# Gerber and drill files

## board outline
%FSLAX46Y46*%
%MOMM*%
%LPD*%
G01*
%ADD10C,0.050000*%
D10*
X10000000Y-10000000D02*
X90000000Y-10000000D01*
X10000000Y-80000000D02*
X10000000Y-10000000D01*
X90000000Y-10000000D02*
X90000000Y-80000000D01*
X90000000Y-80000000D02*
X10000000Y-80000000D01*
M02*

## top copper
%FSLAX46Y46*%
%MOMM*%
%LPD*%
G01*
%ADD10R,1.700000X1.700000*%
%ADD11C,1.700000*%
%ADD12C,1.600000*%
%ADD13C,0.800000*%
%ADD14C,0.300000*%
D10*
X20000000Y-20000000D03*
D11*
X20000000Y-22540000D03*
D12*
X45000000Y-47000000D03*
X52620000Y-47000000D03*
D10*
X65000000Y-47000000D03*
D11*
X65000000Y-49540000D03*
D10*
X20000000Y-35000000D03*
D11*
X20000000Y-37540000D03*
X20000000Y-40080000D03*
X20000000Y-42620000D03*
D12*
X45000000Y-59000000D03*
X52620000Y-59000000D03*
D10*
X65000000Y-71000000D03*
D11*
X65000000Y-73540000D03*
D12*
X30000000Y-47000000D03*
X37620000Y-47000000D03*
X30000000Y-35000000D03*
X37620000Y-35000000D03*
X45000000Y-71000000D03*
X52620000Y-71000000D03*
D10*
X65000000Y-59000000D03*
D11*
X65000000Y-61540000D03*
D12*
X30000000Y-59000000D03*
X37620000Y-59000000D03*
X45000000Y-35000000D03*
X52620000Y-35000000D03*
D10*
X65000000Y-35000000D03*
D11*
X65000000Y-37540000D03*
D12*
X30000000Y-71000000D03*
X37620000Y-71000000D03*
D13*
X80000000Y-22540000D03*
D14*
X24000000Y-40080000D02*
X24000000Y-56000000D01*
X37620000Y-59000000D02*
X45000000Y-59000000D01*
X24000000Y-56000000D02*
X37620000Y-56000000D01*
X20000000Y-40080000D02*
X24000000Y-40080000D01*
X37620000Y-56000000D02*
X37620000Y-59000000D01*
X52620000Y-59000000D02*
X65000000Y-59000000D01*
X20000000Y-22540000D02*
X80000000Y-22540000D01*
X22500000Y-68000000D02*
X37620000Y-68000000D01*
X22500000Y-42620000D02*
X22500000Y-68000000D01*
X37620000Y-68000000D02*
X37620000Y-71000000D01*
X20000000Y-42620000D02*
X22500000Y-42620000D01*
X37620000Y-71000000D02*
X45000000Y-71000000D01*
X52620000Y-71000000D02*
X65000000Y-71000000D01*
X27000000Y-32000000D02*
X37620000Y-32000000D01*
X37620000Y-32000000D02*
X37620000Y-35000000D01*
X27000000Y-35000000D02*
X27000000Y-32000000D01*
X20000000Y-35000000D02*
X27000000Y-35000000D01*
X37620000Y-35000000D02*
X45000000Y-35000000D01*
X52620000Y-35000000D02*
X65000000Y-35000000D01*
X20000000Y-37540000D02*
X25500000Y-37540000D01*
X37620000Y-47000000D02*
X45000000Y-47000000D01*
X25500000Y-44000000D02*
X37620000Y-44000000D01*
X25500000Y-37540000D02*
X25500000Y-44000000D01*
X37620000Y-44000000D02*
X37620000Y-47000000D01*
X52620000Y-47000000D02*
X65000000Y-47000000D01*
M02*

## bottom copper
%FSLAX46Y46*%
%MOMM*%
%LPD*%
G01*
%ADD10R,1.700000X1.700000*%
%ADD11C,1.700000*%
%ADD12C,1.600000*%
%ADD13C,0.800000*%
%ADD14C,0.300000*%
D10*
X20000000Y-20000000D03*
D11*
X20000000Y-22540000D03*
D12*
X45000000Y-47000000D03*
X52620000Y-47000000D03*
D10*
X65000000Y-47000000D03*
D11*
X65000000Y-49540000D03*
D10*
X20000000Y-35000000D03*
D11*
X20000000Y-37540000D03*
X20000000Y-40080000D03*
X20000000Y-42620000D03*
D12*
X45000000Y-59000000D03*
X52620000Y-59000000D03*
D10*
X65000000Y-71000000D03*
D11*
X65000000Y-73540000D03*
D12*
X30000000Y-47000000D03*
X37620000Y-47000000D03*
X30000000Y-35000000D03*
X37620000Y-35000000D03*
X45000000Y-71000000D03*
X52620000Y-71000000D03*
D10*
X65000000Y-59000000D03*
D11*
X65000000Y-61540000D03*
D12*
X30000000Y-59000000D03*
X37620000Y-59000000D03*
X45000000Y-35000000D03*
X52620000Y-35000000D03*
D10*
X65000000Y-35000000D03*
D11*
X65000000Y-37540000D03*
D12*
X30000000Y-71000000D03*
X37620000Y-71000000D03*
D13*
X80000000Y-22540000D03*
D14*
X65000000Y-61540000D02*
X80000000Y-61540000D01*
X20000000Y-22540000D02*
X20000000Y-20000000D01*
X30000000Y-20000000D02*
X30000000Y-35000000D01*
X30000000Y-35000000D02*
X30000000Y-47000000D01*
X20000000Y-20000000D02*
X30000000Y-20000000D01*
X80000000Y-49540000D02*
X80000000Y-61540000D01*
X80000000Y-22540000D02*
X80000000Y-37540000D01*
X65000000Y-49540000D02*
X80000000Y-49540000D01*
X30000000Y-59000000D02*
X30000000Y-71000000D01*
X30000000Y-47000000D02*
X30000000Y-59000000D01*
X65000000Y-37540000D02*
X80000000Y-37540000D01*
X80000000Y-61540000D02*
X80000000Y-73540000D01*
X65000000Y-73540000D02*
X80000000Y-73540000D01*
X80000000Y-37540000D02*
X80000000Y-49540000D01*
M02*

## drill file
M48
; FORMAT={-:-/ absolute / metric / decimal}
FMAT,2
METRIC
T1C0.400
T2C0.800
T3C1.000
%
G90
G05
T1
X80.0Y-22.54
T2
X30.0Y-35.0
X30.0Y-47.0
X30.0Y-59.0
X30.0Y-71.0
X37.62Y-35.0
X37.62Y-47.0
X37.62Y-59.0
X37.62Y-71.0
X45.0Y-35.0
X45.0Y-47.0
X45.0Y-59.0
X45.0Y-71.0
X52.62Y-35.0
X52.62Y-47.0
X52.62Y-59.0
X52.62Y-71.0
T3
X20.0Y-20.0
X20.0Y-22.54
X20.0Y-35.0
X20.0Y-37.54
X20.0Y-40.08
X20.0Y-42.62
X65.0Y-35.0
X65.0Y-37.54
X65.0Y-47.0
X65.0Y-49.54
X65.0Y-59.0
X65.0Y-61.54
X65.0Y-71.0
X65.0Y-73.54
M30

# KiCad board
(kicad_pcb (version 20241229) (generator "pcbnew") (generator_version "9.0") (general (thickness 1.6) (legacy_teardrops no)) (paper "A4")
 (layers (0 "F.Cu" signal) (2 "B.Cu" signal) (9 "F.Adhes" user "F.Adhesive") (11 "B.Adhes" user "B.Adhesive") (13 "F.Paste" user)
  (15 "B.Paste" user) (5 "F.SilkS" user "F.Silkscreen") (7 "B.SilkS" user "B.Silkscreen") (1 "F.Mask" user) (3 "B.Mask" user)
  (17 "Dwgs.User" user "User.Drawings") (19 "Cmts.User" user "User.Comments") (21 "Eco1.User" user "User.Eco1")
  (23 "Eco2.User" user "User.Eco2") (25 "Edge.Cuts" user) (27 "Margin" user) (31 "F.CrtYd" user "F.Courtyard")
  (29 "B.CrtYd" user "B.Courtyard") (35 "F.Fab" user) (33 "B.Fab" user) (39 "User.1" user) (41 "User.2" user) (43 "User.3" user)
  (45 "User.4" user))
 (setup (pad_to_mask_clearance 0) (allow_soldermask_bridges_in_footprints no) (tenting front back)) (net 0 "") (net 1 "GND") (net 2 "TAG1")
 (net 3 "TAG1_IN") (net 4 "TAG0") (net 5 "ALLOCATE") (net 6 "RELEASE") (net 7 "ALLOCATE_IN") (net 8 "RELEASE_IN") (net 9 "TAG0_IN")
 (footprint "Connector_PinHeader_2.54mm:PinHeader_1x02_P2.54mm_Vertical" (layer "F.Cu") (at 20 20)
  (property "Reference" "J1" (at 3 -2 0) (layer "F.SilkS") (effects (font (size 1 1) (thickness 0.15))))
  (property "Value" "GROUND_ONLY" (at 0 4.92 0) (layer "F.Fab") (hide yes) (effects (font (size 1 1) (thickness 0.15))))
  (pad "1" thru_hole rect (at 0 0) (size 1.7 1.7) (drill 1) (layers "*.Cu" "*.Mask") (remove_unused_layers no) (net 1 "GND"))
  (pad "2" thru_hole circle (at 0 2.54) (size 1.7 1.7) (drill 1) (layers "*.Cu" "*.Mask") (remove_unused_layers no) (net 1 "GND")))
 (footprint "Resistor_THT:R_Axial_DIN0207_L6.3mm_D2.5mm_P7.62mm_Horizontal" (layer "F.Cu") (at 45 47)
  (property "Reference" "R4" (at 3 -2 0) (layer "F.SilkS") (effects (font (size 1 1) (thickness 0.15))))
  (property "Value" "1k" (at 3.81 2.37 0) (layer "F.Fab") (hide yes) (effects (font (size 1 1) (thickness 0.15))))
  (pad "1" thru_hole circle (at 0 0) (size 1.6 1.6) (drill 0.8) (layers "*.Cu" "*.Mask") (remove_unused_layers no) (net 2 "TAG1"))
  (pad "2" thru_hole circle (at 7.62 0) (size 1.6 1.6) (drill 0.8) (layers "*.Cu" "*.Mask") (remove_unused_layers no) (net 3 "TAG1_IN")))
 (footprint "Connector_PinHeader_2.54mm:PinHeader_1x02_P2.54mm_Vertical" (layer "F.Cu") (at 65 47)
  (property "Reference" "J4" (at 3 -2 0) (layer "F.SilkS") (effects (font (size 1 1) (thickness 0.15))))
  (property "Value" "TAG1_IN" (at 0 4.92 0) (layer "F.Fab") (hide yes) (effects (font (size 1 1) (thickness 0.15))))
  (pad "1" thru_hole rect (at 0 0) (size 1.7 1.7) (drill 1) (layers "*.Cu" "*.Mask") (remove_unused_layers no) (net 3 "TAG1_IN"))
  (pad "2" thru_hole circle (at 0 2.54) (size 1.7 1.7) (drill 1) (layers "*.Cu" "*.Mask") (remove_unused_layers no) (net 1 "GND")))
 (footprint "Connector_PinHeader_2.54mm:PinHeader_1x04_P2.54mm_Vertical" (layer "F.Cu") (at 20 35)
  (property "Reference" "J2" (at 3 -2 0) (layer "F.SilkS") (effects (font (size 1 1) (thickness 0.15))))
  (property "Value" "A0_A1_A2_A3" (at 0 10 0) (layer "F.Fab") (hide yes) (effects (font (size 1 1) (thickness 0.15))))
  (pad "1" thru_hole rect (at 0 0) (size 1.7 1.7) (drill 1) (layers "*.Cu" "*.Mask") (remove_unused_layers no) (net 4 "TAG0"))
  (pad "2" thru_hole circle (at 0 2.54) (size 1.7 1.7) (drill 1) (layers "*.Cu" "*.Mask") (remove_unused_layers no) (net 2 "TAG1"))
  (pad "3" thru_hole circle (at 0 5.08) (size 1.7 1.7) (drill 1) (layers "*.Cu" "*.Mask") (remove_unused_layers no) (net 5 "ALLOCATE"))
  (pad "4" thru_hole circle (at 0 7.62) (size 1.7 1.7) (drill 1) (layers "*.Cu" "*.Mask") (remove_unused_layers no) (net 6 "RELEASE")))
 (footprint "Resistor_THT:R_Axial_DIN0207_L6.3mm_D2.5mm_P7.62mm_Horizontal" (layer "F.Cu") (at 45 59)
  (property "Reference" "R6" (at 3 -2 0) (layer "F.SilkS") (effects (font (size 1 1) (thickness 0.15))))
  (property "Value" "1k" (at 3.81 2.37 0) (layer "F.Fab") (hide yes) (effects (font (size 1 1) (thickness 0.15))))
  (pad "1" thru_hole circle (at 0 0) (size 1.6 1.6) (drill 0.8) (layers "*.Cu" "*.Mask") (remove_unused_layers no) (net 5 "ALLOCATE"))
  (pad "2" thru_hole circle (at 7.62 0) (size 1.6 1.6) (drill 0.8) (layers "*.Cu" "*.Mask") (remove_unused_layers no) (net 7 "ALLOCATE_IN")))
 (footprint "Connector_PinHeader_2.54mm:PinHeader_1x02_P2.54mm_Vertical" (layer "F.Cu") (at 65 71)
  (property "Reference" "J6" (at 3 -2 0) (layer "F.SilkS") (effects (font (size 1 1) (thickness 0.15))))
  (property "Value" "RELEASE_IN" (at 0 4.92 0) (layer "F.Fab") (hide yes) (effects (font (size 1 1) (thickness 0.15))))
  (pad "1" thru_hole rect (at 0 0) (size 1.7 1.7) (drill 1) (layers "*.Cu" "*.Mask") (remove_unused_layers no) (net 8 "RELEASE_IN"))
  (pad "2" thru_hole circle (at 0 2.54) (size 1.7 1.7) (drill 1) (layers "*.Cu" "*.Mask") (remove_unused_layers no) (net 1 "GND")))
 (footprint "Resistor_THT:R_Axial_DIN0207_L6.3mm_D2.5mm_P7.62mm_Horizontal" (layer "F.Cu") (at 30 47)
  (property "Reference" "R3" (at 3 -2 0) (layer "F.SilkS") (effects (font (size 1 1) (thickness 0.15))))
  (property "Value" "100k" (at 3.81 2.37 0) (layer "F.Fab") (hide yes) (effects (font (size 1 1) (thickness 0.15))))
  (pad "1" thru_hole circle (at 0 0) (size 1.6 1.6) (drill 0.8) (layers "*.Cu" "*.Mask") (remove_unused_layers no) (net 1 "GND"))
  (pad "2" thru_hole circle (at 7.62 0) (size 1.6 1.6) (drill 0.8) (layers "*.Cu" "*.Mask") (remove_unused_layers no) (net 2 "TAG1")))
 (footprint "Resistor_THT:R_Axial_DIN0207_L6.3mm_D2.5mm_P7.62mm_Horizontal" (layer "F.Cu") (at 30 35)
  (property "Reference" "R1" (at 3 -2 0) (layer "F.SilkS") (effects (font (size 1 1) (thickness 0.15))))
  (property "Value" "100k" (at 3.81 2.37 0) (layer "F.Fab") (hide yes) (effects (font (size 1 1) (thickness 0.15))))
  (pad "1" thru_hole circle (at 0 0) (size 1.6 1.6) (drill 0.8) (layers "*.Cu" "*.Mask") (remove_unused_layers no) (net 1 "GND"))
  (pad "2" thru_hole circle (at 7.62 0) (size 1.6 1.6) (drill 0.8) (layers "*.Cu" "*.Mask") (remove_unused_layers no) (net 4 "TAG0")))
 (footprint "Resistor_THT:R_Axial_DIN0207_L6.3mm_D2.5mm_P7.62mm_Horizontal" (layer "F.Cu") (at 45 71)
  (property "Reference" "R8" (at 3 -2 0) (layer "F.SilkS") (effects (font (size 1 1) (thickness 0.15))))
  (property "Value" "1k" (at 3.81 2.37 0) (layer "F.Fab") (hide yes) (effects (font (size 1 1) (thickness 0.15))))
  (pad "1" thru_hole circle (at 0 0) (size 1.6 1.6) (drill 0.8) (layers "*.Cu" "*.Mask") (remove_unused_layers no) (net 6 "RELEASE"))
  (pad "2" thru_hole circle (at 7.62 0) (size 1.6 1.6) (drill 0.8) (layers "*.Cu" "*.Mask") (remove_unused_layers no) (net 8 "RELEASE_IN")))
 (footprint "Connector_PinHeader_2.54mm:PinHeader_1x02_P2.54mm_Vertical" (layer "F.Cu") (at 65 59)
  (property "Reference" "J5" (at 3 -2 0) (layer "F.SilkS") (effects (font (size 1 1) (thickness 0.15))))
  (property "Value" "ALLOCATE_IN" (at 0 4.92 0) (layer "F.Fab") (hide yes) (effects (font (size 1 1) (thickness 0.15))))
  (pad "1" thru_hole rect (at 0 0) (size 1.7 1.7) (drill 1) (layers "*.Cu" "*.Mask") (remove_unused_layers no) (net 7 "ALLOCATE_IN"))
  (pad "2" thru_hole circle (at 0 2.54) (size 1.7 1.7) (drill 1) (layers "*.Cu" "*.Mask") (remove_unused_layers no) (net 1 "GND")))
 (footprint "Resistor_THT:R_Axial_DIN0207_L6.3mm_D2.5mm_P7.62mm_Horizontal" (layer "F.Cu") (at 30 59)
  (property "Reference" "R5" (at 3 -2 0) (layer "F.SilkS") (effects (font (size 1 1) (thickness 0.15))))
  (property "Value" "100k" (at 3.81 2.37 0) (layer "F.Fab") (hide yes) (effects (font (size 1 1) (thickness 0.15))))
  (pad "1" thru_hole circle (at 0 0) (size 1.6 1.6) (drill 0.8) (layers "*.Cu" "*.Mask") (remove_unused_layers no) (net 1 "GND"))
  (pad "2" thru_hole circle (at 7.62 0) (size 1.6 1.6) (drill 0.8) (layers "*.Cu" "*.Mask") (remove_unused_layers no) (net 5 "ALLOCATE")))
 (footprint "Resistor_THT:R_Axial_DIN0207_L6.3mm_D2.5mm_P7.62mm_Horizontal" (layer "F.Cu") (at 45 35)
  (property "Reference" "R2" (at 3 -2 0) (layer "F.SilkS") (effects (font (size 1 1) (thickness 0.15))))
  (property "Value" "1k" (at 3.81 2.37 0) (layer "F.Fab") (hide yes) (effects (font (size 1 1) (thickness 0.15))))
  (pad "1" thru_hole circle (at 0 0) (size 1.6 1.6) (drill 0.8) (layers "*.Cu" "*.Mask") (remove_unused_layers no) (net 4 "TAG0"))
  (pad "2" thru_hole circle (at 7.62 0) (size 1.6 1.6) (drill 0.8) (layers "*.Cu" "*.Mask") (remove_unused_layers no) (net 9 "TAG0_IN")))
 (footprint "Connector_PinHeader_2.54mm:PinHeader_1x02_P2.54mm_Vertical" (layer "F.Cu") (at 65 35)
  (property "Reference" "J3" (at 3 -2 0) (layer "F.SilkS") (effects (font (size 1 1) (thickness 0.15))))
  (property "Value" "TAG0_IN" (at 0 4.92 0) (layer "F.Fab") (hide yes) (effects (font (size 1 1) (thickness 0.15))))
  (pad "1" thru_hole rect (at 0 0) (size 1.7 1.7) (drill 1) (layers "*.Cu" "*.Mask") (remove_unused_layers no) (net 9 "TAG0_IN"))
  (pad "2" thru_hole circle (at 0 2.54) (size 1.7 1.7) (drill 1) (layers "*.Cu" "*.Mask") (remove_unused_layers no) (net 1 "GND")))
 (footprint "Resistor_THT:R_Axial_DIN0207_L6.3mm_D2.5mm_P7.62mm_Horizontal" (layer "F.Cu") (at 30 71)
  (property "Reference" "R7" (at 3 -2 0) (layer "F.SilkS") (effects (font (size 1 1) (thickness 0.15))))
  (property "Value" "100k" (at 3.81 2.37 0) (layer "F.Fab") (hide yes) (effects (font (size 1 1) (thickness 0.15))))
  (pad "1" thru_hole circle (at 0 0) (size 1.6 1.6) (drill 0.8) (layers "*.Cu" "*.Mask") (remove_unused_layers no) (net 1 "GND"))
  (pad "2" thru_hole circle (at 7.62 0) (size 1.6 1.6) (drill 0.8) (layers "*.Cu" "*.Mask") (remove_unused_layers no) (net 6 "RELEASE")))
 (gr_line (start 10 10) (end 90 10) (stroke (width 0.05) (type default)) (layer "Edge.Cuts"))
 (gr_line (start 10 80) (end 10 10) (stroke (width 0.05) (type default)) (layer "Edge.Cuts"))
 (gr_line (start 90 10) (end 90 80) (stroke (width 0.05) (type default)) (layer "Edge.Cuts"))
 (gr_line (start 90 80) (end 10 80) (stroke (width 0.05) (type default)) (layer "Edge.Cuts"))
 (segment (start 24 40.08) (end 24 56) (width 0.3) (layer "F.Cu") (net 5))
 (segment (start 37.62 59) (end 45 59) (width 0.3) (layer "F.Cu") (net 5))
 (segment (start 24 56) (end 37.62 56) (width 0.3) (layer "F.Cu") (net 5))
 (segment (start 20 40.08) (end 24 40.08) (width 0.3) (layer "F.Cu") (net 5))
 (segment (start 37.62 56) (end 37.62 59) (width 0.3) (layer "F.Cu") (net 5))
 (segment (start 52.62 59) (end 65 59) (width 0.3) (layer "F.Cu") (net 7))
 (segment (start 20 22.54) (end 80 22.54) (width 0.3) (layer "F.Cu") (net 1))
 (via (at 80 22.54) (size 0.8) (drill 0.4) (layers "F.Cu" "B.Cu") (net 1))
 (segment (start 65 61.54) (end 80 61.54) (width 0.3) (layer "B.Cu") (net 1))
 (segment (start 20 22.54) (end 20 20) (width 0.3) (layer "B.Cu") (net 1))
 (segment (start 30 20) (end 30 35) (width 0.3) (layer "B.Cu") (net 1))
 (segment (start 30 35) (end 30 47) (width 0.3) (layer "B.Cu") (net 1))
 (segment (start 20 20) (end 30 20) (width 0.3) (layer "B.Cu") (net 1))
 (segment (start 80 49.54) (end 80 61.54) (width 0.3) (layer "B.Cu") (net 1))
 (segment (start 80 22.54) (end 80 37.54) (width 0.3) (layer "B.Cu") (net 1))
 (segment (start 65 49.54) (end 80 49.54) (width 0.3) (layer "B.Cu") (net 1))
 (segment (start 30 59) (end 30 71) (width 0.3) (layer "B.Cu") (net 1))
 (segment (start 30 47) (end 30 59) (width 0.3) (layer "B.Cu") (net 1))
 (segment (start 65 37.54) (end 80 37.54) (width 0.3) (layer "B.Cu") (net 1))
 (segment (start 80 61.54) (end 80 73.54) (width 0.3) (layer "B.Cu") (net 1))
 (segment (start 65 73.54) (end 80 73.54) (width 0.3) (layer "B.Cu") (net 1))
 (segment (start 80 37.54) (end 80 49.54) (width 0.3) (layer "B.Cu") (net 1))
 (segment (start 22.5 68) (end 37.62 68) (width 0.3) (layer "F.Cu") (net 6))
 (segment (start 22.5 42.62) (end 22.5 68) (width 0.3) (layer "F.Cu") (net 6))
 (segment (start 37.62 68) (end 37.62 71) (width 0.3) (layer "F.Cu") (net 6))
 (segment (start 20 42.62) (end 22.5 42.62) (width 0.3) (layer "F.Cu") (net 6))
 (segment (start 37.62 71) (end 45 71) (width 0.3) (layer "F.Cu") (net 6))
 (segment (start 52.62 71) (end 65 71) (width 0.3) (layer "F.Cu") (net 8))
 (segment (start 27 32) (end 37.62 32) (width 0.3) (layer "F.Cu") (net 4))
 (segment (start 37.62 32) (end 37.62 35) (width 0.3) (layer "F.Cu") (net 4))
 (segment (start 27 35) (end 27 32) (width 0.3) (layer "F.Cu") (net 4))
 (segment (start 20 35) (end 27 35) (width 0.3) (layer "F.Cu") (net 4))
 (segment (start 37.62 35) (end 45 35) (width 0.3) (layer "F.Cu") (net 4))
 (segment (start 52.62 35) (end 65 35) (width 0.3) (layer "F.Cu") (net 9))
 (segment (start 20 37.54) (end 25.5 37.54) (width 0.3) (layer "F.Cu") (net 2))
 (segment (start 37.62 47) (end 45 47) (width 0.3) (layer "F.Cu") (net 2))
 (segment (start 25.5 44) (end 37.62 44) (width 0.3) (layer "F.Cu") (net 2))
 (segment (start 25.5 37.54) (end 25.5 44) (width 0.3) (layer "F.Cu") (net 2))
 (segment (start 37.62 44) (end 37.62 47) (width 0.3) (layer "F.Cu") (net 2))
 (segment (start 52.62 47) (end 65 47) (width 0.3) (layer "F.Cu") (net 3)))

